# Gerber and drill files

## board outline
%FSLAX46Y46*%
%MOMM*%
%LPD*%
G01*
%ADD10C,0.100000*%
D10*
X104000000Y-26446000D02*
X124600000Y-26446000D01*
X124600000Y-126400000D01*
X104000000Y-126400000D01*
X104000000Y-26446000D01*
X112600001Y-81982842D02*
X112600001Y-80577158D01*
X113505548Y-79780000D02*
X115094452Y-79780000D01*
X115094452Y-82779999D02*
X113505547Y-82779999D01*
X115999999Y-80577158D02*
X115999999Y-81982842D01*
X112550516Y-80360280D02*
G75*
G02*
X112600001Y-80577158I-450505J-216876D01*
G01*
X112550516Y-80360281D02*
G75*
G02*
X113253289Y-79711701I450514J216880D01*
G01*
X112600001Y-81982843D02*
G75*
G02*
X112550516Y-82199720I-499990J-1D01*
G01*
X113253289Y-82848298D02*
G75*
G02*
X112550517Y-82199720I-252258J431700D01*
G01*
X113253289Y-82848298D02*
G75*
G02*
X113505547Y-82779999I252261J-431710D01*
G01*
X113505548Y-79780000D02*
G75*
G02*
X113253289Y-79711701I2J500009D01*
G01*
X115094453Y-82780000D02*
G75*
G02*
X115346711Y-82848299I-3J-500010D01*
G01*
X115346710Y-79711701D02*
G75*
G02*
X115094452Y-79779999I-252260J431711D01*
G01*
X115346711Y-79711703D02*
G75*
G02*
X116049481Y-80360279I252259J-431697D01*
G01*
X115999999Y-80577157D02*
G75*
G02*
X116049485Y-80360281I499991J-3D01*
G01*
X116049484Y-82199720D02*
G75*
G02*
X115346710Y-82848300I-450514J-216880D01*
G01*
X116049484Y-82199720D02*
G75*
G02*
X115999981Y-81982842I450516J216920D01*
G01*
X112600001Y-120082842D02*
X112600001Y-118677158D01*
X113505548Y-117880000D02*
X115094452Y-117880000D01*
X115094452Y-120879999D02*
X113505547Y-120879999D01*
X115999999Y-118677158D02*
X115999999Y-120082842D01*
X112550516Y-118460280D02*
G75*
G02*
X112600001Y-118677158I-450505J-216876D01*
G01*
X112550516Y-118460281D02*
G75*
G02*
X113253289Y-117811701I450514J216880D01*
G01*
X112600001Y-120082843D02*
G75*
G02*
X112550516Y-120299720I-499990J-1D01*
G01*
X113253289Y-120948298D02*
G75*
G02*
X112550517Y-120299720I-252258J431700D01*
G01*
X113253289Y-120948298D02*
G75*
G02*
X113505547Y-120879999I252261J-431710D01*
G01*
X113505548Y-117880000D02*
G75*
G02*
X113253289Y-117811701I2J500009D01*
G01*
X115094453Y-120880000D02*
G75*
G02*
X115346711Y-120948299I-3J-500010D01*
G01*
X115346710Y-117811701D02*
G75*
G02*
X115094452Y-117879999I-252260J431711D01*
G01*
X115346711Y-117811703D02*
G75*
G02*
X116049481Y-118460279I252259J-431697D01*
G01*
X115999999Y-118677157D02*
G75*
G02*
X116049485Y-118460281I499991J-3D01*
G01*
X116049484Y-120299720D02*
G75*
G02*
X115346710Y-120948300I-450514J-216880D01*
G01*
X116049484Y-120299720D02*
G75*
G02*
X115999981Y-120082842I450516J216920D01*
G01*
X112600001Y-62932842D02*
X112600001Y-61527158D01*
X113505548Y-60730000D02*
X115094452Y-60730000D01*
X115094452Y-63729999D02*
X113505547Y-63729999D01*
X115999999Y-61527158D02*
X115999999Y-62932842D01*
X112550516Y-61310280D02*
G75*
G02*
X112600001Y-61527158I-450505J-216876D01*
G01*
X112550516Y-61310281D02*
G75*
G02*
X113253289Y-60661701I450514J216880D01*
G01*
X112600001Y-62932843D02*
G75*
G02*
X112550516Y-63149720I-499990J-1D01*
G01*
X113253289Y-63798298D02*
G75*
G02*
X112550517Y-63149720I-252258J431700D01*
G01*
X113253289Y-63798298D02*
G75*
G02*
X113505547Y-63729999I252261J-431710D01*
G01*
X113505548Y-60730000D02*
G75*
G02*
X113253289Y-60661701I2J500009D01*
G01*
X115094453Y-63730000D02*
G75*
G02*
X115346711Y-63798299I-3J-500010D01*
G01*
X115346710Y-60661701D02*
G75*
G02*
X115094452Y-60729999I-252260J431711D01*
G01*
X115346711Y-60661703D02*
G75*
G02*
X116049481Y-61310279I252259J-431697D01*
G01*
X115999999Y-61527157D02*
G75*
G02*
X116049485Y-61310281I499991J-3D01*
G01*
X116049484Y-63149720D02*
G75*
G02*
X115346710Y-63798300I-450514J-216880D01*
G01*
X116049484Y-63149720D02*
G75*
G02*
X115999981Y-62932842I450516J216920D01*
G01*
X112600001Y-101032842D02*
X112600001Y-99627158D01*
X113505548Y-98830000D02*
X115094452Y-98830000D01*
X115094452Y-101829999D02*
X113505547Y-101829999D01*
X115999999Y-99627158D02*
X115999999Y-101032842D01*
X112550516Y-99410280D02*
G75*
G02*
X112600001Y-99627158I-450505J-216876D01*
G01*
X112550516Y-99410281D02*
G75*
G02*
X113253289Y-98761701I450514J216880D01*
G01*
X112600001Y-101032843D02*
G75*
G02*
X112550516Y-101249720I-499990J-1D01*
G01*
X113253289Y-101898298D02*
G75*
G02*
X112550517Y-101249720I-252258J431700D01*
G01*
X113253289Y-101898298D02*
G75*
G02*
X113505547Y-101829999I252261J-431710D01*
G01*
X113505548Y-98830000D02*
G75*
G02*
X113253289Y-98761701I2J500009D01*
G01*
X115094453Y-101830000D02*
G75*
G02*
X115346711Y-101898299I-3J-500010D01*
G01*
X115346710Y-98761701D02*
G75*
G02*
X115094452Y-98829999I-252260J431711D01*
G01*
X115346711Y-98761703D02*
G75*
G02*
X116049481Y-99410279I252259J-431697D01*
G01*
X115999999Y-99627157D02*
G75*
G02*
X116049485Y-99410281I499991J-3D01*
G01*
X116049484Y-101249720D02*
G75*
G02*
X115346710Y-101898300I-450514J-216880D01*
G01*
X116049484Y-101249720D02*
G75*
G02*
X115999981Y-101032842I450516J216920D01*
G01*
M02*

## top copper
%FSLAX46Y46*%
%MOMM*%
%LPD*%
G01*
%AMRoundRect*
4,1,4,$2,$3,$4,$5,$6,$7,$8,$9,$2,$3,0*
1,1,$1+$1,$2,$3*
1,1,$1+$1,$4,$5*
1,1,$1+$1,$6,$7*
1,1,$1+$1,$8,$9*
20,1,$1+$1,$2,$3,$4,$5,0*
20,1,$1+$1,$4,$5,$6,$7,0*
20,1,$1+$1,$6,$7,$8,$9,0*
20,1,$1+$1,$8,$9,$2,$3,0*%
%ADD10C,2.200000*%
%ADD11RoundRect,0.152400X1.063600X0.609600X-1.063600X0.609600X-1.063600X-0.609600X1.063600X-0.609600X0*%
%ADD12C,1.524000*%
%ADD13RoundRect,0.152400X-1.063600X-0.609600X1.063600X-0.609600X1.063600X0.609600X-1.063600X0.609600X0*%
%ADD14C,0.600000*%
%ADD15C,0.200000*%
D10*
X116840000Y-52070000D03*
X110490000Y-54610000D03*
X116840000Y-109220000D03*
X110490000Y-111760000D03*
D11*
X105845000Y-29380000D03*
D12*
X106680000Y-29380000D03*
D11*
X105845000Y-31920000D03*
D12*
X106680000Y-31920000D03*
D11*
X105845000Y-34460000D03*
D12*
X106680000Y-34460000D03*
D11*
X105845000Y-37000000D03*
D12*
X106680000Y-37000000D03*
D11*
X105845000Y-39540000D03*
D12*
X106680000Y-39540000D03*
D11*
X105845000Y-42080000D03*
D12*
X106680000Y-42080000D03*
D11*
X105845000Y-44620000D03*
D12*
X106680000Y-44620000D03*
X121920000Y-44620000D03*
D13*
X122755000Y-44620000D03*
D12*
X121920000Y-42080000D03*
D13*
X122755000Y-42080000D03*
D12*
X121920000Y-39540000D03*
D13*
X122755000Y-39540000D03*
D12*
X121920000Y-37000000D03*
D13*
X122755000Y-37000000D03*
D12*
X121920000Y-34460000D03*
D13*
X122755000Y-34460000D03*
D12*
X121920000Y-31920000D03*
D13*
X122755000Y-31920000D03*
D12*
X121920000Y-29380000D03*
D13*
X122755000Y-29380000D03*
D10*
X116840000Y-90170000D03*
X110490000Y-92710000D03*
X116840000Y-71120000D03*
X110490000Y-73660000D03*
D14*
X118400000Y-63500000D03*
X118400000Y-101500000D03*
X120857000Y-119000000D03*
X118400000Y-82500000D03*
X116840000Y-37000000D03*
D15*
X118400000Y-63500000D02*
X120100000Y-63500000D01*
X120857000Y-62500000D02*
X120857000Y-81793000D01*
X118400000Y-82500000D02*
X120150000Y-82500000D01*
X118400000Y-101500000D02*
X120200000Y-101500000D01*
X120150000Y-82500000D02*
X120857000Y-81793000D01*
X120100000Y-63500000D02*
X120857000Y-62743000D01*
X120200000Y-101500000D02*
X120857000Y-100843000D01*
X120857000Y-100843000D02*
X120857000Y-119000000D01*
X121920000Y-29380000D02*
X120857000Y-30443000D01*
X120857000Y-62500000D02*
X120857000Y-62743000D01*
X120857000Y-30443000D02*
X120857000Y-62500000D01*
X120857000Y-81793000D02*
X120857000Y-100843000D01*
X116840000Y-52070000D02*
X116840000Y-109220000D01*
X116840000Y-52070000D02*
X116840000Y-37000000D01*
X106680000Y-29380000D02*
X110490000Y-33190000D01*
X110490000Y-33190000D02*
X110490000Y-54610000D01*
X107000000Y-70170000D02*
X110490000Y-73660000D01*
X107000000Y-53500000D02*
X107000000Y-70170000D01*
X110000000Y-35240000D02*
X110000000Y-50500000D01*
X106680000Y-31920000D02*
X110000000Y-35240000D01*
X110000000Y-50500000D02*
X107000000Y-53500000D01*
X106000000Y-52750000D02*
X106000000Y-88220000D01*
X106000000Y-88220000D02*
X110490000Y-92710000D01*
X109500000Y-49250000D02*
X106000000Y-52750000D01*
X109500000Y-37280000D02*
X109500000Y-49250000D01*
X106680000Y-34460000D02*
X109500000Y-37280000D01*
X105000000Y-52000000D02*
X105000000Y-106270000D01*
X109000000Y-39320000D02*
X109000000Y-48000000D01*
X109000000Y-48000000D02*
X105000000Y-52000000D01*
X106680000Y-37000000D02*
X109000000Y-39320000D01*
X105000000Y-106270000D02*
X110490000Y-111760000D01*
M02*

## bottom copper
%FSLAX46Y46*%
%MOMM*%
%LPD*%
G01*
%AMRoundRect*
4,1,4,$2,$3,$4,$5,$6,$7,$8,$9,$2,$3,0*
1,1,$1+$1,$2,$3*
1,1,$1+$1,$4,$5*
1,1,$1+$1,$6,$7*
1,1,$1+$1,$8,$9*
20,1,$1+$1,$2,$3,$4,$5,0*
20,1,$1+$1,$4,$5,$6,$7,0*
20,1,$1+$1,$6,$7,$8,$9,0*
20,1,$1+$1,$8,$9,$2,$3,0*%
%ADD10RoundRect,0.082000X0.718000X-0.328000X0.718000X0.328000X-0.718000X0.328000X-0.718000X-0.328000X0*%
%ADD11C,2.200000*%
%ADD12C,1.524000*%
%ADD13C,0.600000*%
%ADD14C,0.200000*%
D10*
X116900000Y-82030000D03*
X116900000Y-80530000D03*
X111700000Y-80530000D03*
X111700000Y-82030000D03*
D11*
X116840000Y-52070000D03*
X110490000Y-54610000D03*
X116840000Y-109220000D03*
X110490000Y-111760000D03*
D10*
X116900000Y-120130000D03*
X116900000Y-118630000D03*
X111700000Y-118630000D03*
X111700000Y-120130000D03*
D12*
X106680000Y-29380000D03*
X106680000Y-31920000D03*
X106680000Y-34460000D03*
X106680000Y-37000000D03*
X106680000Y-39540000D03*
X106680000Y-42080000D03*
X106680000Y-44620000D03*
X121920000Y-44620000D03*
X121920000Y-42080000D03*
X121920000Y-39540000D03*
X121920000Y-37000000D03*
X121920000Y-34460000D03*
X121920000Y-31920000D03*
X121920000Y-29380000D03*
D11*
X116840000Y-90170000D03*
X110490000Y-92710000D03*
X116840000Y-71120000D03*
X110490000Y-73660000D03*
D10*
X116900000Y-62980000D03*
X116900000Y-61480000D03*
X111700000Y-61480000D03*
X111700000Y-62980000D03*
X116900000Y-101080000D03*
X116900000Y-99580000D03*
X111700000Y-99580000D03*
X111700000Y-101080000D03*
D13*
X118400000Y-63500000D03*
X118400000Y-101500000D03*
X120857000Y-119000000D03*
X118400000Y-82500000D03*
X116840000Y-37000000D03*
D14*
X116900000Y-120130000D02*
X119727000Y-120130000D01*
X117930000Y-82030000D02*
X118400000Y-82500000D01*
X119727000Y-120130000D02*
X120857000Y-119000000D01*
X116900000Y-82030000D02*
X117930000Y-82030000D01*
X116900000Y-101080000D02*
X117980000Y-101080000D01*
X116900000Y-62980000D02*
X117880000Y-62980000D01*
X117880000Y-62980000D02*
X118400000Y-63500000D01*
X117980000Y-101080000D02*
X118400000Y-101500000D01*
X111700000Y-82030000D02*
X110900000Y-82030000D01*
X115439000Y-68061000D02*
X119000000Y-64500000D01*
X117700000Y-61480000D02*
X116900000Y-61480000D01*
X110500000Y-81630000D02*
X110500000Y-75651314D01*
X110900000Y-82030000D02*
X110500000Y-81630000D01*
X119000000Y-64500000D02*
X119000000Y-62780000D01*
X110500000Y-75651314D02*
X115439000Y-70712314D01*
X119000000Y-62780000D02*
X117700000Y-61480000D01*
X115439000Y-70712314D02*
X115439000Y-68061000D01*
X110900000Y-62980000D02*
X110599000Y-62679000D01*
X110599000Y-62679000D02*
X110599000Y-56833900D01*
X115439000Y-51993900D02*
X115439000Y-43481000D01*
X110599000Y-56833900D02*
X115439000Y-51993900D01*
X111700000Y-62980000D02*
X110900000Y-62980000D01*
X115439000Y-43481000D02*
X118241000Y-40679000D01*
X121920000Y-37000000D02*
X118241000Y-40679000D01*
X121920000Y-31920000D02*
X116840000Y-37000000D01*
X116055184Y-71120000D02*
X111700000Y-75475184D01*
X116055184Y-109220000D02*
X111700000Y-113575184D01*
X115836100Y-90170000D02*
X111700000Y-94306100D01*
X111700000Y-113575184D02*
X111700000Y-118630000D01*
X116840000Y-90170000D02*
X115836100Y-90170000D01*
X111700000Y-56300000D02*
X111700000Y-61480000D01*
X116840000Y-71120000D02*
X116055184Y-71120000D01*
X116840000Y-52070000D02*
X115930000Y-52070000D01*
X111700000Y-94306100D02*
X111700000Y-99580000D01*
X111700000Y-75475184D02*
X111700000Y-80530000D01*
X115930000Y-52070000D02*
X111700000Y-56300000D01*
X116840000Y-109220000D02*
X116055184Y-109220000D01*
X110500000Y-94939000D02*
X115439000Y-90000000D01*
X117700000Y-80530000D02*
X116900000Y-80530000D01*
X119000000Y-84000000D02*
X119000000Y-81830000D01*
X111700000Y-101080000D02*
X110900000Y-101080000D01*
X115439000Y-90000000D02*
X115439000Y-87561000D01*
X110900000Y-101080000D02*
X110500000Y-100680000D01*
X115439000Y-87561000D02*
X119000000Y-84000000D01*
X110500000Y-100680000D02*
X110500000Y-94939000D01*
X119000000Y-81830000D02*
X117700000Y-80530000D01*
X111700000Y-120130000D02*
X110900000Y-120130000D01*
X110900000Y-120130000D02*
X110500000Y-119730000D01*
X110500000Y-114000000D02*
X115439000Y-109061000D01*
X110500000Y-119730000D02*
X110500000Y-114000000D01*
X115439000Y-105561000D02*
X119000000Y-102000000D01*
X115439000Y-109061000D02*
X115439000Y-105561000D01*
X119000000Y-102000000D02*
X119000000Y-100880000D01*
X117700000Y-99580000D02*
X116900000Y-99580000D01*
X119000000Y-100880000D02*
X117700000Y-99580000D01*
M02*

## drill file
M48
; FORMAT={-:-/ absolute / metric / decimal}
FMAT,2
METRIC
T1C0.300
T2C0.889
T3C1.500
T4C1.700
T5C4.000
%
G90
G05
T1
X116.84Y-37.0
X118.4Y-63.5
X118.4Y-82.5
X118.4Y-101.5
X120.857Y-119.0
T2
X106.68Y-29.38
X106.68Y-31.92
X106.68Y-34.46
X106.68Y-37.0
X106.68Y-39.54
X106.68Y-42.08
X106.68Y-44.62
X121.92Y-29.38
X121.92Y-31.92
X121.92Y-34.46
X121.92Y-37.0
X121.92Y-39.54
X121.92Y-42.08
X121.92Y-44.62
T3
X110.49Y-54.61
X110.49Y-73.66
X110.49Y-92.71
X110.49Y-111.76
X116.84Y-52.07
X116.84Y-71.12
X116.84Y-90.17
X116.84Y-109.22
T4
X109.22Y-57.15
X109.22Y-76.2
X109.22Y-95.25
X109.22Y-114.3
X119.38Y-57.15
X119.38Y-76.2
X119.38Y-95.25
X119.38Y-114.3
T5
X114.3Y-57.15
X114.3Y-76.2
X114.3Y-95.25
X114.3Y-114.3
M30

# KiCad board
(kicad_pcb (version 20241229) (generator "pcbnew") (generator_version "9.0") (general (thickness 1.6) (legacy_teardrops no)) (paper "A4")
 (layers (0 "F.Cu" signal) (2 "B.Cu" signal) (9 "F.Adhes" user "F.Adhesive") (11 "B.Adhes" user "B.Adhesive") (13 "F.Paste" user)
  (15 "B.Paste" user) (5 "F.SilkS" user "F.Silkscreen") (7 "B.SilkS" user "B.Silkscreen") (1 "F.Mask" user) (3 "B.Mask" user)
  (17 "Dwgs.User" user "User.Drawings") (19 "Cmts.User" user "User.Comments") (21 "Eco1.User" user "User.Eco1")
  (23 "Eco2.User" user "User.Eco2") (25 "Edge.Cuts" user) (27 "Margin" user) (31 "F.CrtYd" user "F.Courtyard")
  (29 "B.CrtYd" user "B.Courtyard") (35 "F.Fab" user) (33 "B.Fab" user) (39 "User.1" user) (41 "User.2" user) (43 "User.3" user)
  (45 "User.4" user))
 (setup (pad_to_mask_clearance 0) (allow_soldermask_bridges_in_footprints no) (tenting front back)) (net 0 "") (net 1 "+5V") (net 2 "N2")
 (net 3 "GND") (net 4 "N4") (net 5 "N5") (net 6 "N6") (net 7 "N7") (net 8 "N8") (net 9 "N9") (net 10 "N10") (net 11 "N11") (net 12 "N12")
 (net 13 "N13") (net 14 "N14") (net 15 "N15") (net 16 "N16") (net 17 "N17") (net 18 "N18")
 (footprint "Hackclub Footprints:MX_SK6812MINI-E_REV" (layer "F.Cu") (at 114.3 76.2)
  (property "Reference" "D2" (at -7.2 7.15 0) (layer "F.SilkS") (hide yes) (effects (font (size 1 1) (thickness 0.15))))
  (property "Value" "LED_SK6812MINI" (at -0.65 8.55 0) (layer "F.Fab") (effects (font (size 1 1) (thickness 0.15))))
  (fp_line (start -1.699999 5.782842) (end -1.699999 4.377158) (stroke (width 0.1) (type solid)) (layer "Edge.Cuts"))
  (fp_line (start -0.794452 3.58) (end 0.794452 3.58) (stroke (width 0.1) (type solid)) (layer "Edge.Cuts"))
  (fp_line (start 0.794452 6.579999) (end -0.794453 6.579999) (stroke (width 0.1) (type solid)) (layer "Edge.Cuts"))
  (fp_line (start 1.699999 4.377158) (end 1.699999 5.782842) (stroke (width 0.1) (type solid)) (layer "Edge.Cuts"))
  (fp_arc (start -1.749484 4.16028) (mid -1.712527 4.265932) (end -1.699999 4.377158) (stroke (width 0.1) (type solid)) (layer "Edge.Cuts"))
  (fp_arc (start -1.749484 4.160281) (mid -1.638072 3.575965) (end -1.046711 3.511701) (stroke (width 0.1) (type solid)) (layer "Edge.Cuts"))
  (fp_arc (start -1.699999 5.782843) (mid -1.712527 5.894068) (end -1.749484 5.99972) (stroke (width 0.1) (type solid)) (layer "Edge.Cuts"))
  (fp_arc (start -1.046711 6.648298) (mid -1.638071 6.584034) (end -1.749484 5.99972) (stroke (width 0.1) (type solid)) (layer "Edge.Cuts"))
  (fp_arc (start -1.046711 6.648298) (mid -0.925123 6.597376) (end -0.794453 6.579999) (stroke (width 0.1) (type solid)) (layer "Edge.Cuts"))
  (fp_arc (start -0.794452 3.58) (mid -0.925123 3.562623) (end -1.046711 3.511701) (stroke (width 0.1) (type solid)) (layer "Edge.Cuts"))
  (fp_arc (start 0.794453 6.58) (mid 0.925123 6.597377) (end 1.046711 6.648299) (stroke (width 0.1) (type solid)) (layer "Edge.Cuts"))
  (fp_arc (start 1.04671 3.511701) (mid 0.925122 3.562623) (end 0.794452 3.58) (stroke (width 0.1) (type solid)) (layer "Edge.Cuts"))
  (fp_arc (start 1.046711 3.511703) (mid 1.63807 3.575966) (end 1.749484 4.16028) (stroke (width 0.1) (type solid)) (layer "Edge.Cuts"))
  (fp_arc (start 1.699999 4.377157) (mid 1.712527 4.265932) (end 1.749484 4.16028) (stroke (width 0.1) (type solid)) (layer "Edge.Cuts"))
  (fp_arc (start 1.749484 5.99972) (mid 1.638071 6.584035) (end 1.046711 6.648299) (stroke (width 0.1) (type solid)) (layer "Edge.Cuts"))
  (fp_arc (start 1.749484 5.99972) (mid 1.712527 5.894068) (end 1.699999 5.782842) (stroke (width 0.1) (type solid)) (layer "Edge.Cuts"))
  (pad "1" smd roundrect (at 2.6 5.83 90) (size 0.82 1.6) (layers "B.Cu" "B.Mask" "B.Paste") (roundrect_rratio 0.1) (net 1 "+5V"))
  (pad "2" smd roundrect (at 2.6 4.33 90) (size 0.82 1.6) (layers "B.Cu" "B.Mask" "B.Paste") (roundrect_rratio 0.1) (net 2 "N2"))
  (pad "3" smd roundrect (at -2.6 4.33 90) (size 0.82 1.6) (layers "B.Cu" "B.Mask" "B.Paste") (roundrect_rratio 0.1) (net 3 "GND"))
  (pad "4" smd roundrect (at -2.6 5.83 90) (size 0.82 1.6) (layers "B.Cu" "B.Mask" "B.Paste") (roundrect_rratio 0.1) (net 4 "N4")))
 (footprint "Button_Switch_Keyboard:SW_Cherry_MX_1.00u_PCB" (layer "F.Cu") (at 116.84 52.07)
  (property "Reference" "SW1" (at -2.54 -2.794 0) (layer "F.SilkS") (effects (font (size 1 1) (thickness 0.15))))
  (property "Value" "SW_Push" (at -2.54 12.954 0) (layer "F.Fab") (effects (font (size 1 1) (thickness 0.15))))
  (pad "" np_thru_hole circle (at -7.62 5.08) (size 1.7 1.7) (drill 1.7) (layers "*.Cu" "*.Mask"))
  (pad "" np_thru_hole circle (at -2.54 5.08) (size 4 4) (drill 4) (layers "*.Cu" "*.Mask"))
  (pad "" np_thru_hole circle (at 2.54 5.08) (size 1.7 1.7) (drill 1.7) (layers "*.Cu" "*.Mask"))
  (pad "1" thru_hole circle (at 0 0) (size 2.2 2.2) (drill 1.5) (layers "*.Cu" "*.Mask") (remove_unused_layers no) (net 3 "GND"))
  (pad "2" thru_hole circle (at -6.35 2.54) (size 2.2 2.2) (drill 1.5) (layers "*.Cu" "*.Mask") (remove_unused_layers no) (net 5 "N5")))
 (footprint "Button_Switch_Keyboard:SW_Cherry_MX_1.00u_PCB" (layer "F.Cu") (at 116.84 109.22)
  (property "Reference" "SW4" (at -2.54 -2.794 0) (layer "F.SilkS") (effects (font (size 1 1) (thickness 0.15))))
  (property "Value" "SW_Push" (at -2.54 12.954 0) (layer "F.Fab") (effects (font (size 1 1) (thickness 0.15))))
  (pad "" np_thru_hole circle (at -7.62 5.08) (size 1.7 1.7) (drill 1.7) (layers "*.Cu" "*.Mask"))
  (pad "" np_thru_hole circle (at -2.54 5.08) (size 4 4) (drill 4) (layers "*.Cu" "*.Mask"))
  (pad "" np_thru_hole circle (at 2.54 5.08) (size 1.7 1.7) (drill 1.7) (layers "*.Cu" "*.Mask"))
  (pad "1" thru_hole circle (at 0 0) (size 2.2 2.2) (drill 1.5) (layers "*.Cu" "*.Mask") (remove_unused_layers no) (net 3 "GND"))
  (pad "2" thru_hole circle (at -6.35 2.54) (size 2.2 2.2) (drill 1.5) (layers "*.Cu" "*.Mask") (remove_unused_layers no) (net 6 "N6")))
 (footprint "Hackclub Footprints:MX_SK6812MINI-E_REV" (layer "F.Cu") (at 114.3 114.3)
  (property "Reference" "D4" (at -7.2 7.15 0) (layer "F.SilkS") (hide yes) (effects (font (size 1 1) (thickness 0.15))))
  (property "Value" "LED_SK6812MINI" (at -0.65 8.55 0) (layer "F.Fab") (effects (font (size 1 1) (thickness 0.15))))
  (fp_line (start -1.699999 5.782842) (end -1.699999 4.377158) (stroke (width 0.1) (type solid)) (layer "Edge.Cuts"))
  (fp_line (start -0.794452 3.58) (end 0.794452 3.58) (stroke (width 0.1) (type solid)) (layer "Edge.Cuts"))
  (fp_line (start 0.794452 6.579999) (end -0.794453 6.579999) (stroke (width 0.1) (type solid)) (layer "Edge.Cuts"))
  (fp_line (start 1.699999 4.377158) (end 1.699999 5.782842) (stroke (width 0.1) (type solid)) (layer "Edge.Cuts"))
  (fp_arc (start -1.749484 4.16028) (mid -1.712527 4.265932) (end -1.699999 4.377158) (stroke (width 0.1) (type solid)) (layer "Edge.Cuts"))
  (fp_arc (start -1.749484 4.160281) (mid -1.638072 3.575965) (end -1.046711 3.511701) (stroke (width 0.1) (type solid)) (layer "Edge.Cuts"))
  (fp_arc (start -1.699999 5.782843) (mid -1.712527 5.894068) (end -1.749484 5.99972) (stroke (width 0.1) (type solid)) (layer "Edge.Cuts"))
  (fp_arc (start -1.046711 6.648298) (mid -1.638071 6.584034) (end -1.749484 5.99972) (stroke (width 0.1) (type solid)) (layer "Edge.Cuts"))
  (fp_arc (start -1.046711 6.648298) (mid -0.925123 6.597376) (end -0.794453 6.579999) (stroke (width 0.1) (type solid)) (layer "Edge.Cuts"))
  (fp_arc (start -0.794452 3.58) (mid -0.925123 3.562623) (end -1.046711 3.511701) (stroke (width 0.1) (type solid)) (layer "Edge.Cuts"))
  (fp_arc (start 0.794453 6.58) (mid 0.925123 6.597377) (end 1.046711 6.648299) (stroke (width 0.1) (type solid)) (layer "Edge.Cuts"))
  (fp_arc (start 1.04671 3.511701) (mid 0.925122 3.562623) (end 0.794452 3.58) (stroke (width 0.1) (type solid)) (layer "Edge.Cuts"))
  (fp_arc (start 1.046711 3.511703) (mid 1.63807 3.575966) (end 1.749484 4.16028) (stroke (width 0.1) (type solid)) (layer "Edge.Cuts"))
  (fp_arc (start 1.699999 4.377157) (mid 1.712527 4.265932) (end 1.749484 4.16028) (stroke (width 0.1) (type solid)) (layer "Edge.Cuts"))
  (fp_arc (start 1.749484 5.99972) (mid 1.638071 6.584035) (end 1.046711 6.648299) (stroke (width 0.1) (type solid)) (layer "Edge.Cuts"))
  (fp_arc (start 1.749484 5.99972) (mid 1.712527 5.894068) (end 1.699999 5.782842) (stroke (width 0.1) (type solid)) (layer "Edge.Cuts"))
  (pad "1" smd roundrect (at 2.6 5.83 90) (size 0.82 1.6) (layers "B.Cu" "B.Mask" "B.Paste") (roundrect_rratio 0.1) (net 1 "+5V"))
  (pad "2" smd roundrect (at 2.6 4.33 90) (size 0.82 1.6) (layers "B.Cu" "B.Mask" "B.Paste") (roundrect_rratio 0.1) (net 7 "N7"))
  (pad "3" smd roundrect (at -2.6 4.33 90) (size 0.82 1.6) (layers "B.Cu" "B.Mask" "B.Paste") (roundrect_rratio 0.1) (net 3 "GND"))
  (pad "4" smd roundrect (at -2.6 5.83 90) (size 0.82 1.6) (layers "B.Cu" "B.Mask" "B.Paste") (roundrect_rratio 0.1) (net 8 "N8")))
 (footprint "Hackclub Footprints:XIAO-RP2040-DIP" (layer "F.Cu") (at 114.3 37)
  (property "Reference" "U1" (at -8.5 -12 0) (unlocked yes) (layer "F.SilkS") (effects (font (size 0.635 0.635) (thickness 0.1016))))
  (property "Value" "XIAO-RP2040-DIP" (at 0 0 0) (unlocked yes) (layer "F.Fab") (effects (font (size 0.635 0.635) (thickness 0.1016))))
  (pad "1" smd roundrect (at -8.455 -7.62 180) (size 2.432 1.524) (layers "F.Cu" "F.Mask") (roundrect_rratio 0.1) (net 5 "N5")
   (thermal_bridge_angle 45))
  (pad "1" thru_hole circle (at -7.62 -7.62 180) (size 1.524 1.524) (drill 0.889) (layers "*.Cu" "*.Mask") (remove_unused_layers no)
   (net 5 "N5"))
  (pad "2" smd roundrect (at -8.455 -5.08 180) (size 2.432 1.524) (layers "F.Cu" "F.Mask") (roundrect_rratio 0.1) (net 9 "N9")
   (thermal_bridge_angle 45))
  (pad "2" thru_hole circle (at -7.62 -5.08 180) (size 1.524 1.524) (drill 0.889) (layers "*.Cu" "*.Mask") (remove_unused_layers no)
   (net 9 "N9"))
  (pad "3" smd roundrect (at -8.455 -2.54 180) (size 2.432 1.524) (layers "F.Cu" "F.Mask") (roundrect_rratio 0.1) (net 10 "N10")
   (thermal_bridge_angle 45))
  (pad "3" thru_hole circle (at -7.62 -2.54 180) (size 1.524 1.524) (drill 0.889) (layers "*.Cu" "*.Mask") (remove_unused_layers no)
   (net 10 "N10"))
  (pad "4" smd roundrect (at -8.455 0 180) (size 2.432 1.524) (layers "F.Cu" "F.Mask") (roundrect_rratio 0.1) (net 6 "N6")
   (thermal_bridge_angle 45))
  (pad "4" thru_hole circle (at -7.62 0 180) (size 1.524 1.524) (drill 0.889) (layers "*.Cu" "*.Mask") (remove_unused_layers no)
   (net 6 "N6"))
  (pad "5" smd roundrect (at -8.455 2.54 180) (size 2.432 1.524) (layers "F.Cu" "F.Mask") (roundrect_rratio 0.1) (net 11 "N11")
   (thermal_bridge_angle 45))
  (pad "5" thru_hole circle (at -7.62 2.54 180) (size 1.524 1.524) (drill 0.889) (layers "*.Cu" "*.Mask") (remove_unused_layers no)
   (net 11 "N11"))
  (pad "6" smd roundrect (at -8.455 5.08 180) (size 2.432 1.524) (layers "F.Cu" "F.Mask") (roundrect_rratio 0.1) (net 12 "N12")
   (thermal_bridge_angle 45))
  (pad "6" thru_hole circle (at -7.62 5.08 180) (size 1.524 1.524) (drill 0.889) (layers "*.Cu" "*.Mask") (remove_unused_layers no)
   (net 12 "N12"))
  (pad "7" smd roundrect (at -8.455 7.62 180) (size 2.432 1.524) (layers "F.Cu" "F.Mask") (roundrect_rratio 0.1) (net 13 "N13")
   (thermal_bridge_angle 45))
  (pad "7" thru_hole circle (at -7.62 7.62 180) (size 1.524 1.524) (drill 0.889) (layers "*.Cu" "*.Mask") (remove_unused_layers no)
   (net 13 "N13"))
  (pad "8" thru_hole circle (at 7.62 7.62) (size 1.524 1.524) (drill 0.889) (layers "*.Cu" "*.Mask") (remove_unused_layers no)
   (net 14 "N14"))
  (pad "8" smd roundrect (at 8.455 7.62) (size 2.432 1.524) (layers "F.Cu" "F.Mask") (roundrect_rratio 0.1) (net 14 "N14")
   (thermal_bridge_angle 45))
  (pad "9" thru_hole circle (at 7.62 5.08) (size 1.524 1.524) (drill 0.889) (layers "*.Cu" "*.Mask") (remove_unused_layers no)
   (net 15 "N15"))
  (pad "9" smd roundrect (at 8.455 5.08) (size 2.432 1.524) (layers "F.Cu" "F.Mask") (roundrect_rratio 0.1) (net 15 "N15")
   (thermal_bridge_angle 45))
  (pad "10" thru_hole circle (at 7.62 2.54) (size 1.524 1.524) (drill 0.889) (layers "*.Cu" "*.Mask") (remove_unused_layers no)
   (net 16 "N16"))
  (pad "10" smd roundrect (at 8.455 2.54) (size 2.432 1.524) (layers "F.Cu" "F.Mask") (roundrect_rratio 0.1) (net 16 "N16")
   (thermal_bridge_angle 45))
  (pad "11" thru_hole circle (at 7.62 0) (size 1.524 1.524) (drill 0.889) (layers "*.Cu" "*.Mask") (remove_unused_layers no) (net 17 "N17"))
  (pad "11" smd roundrect (at 8.455 0) (size 2.432 1.524) (layers "F.Cu" "F.Mask") (roundrect_rratio 0.1) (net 17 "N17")
   (thermal_bridge_angle 45))
  (pad "12" thru_hole circle (at 7.62 -2.54) (size 1.524 1.524) (drill 0.889) (layers "*.Cu" "*.Mask") (remove_unused_layers no)
   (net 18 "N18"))
  (pad "12" smd roundrect (at 8.455 -2.54) (size 2.432 1.524) (layers "F.Cu" "F.Mask") (roundrect_rratio 0.1) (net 18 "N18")
   (thermal_bridge_angle 45))
  (pad "13" thru_hole circle (at 7.62 -5.08) (size 1.524 1.524) (drill 0.889) (layers "*.Cu" "*.Mask") (remove_unused_layers no)
   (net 3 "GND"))
  (pad "13" smd roundrect (at 8.455 -5.08) (size 2.432 1.524) (layers "F.Cu" "F.Mask") (roundrect_rratio 0.1) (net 3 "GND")
   (thermal_bridge_angle 45))
  (pad "14" thru_hole circle (at 7.62 -7.62) (size 1.524 1.524) (drill 0.889) (layers "*.Cu" "*.Mask") (remove_unused_layers no)
   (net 1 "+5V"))
  (pad "14" smd roundrect (at 8.455 -7.62) (size 2.432 1.524) (layers "F.Cu" "F.Mask") (roundrect_rratio 0.1) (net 1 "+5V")
   (thermal_bridge_angle 45)))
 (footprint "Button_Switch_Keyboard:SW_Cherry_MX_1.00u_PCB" (layer "F.Cu") (at 116.84 90.17)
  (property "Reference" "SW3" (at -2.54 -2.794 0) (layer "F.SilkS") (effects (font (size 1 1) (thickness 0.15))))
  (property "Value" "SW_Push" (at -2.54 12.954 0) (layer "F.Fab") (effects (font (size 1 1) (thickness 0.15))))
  (pad "" np_thru_hole circle (at -7.62 5.08) (size 1.7 1.7) (drill 1.7) (layers "*.Cu" "*.Mask"))
  (pad "" np_thru_hole circle (at -2.54 5.08) (size 4 4) (drill 4) (layers "*.Cu" "*.Mask"))
  (pad "" np_thru_hole circle (at 2.54 5.08) (size 1.7 1.7) (drill 1.7) (layers "*.Cu" "*.Mask"))
  (pad "1" thru_hole circle (at 0 0) (size 2.2 2.2) (drill 1.5) (layers "*.Cu" "*.Mask") (remove_unused_layers no) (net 3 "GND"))
  (pad "2" thru_hole circle (at -6.35 2.54) (size 2.2 2.2) (drill 1.5) (layers "*.Cu" "*.Mask") (remove_unused_layers no) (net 10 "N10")))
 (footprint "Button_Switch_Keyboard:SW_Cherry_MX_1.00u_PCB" (layer "F.Cu") (at 116.84 71.12)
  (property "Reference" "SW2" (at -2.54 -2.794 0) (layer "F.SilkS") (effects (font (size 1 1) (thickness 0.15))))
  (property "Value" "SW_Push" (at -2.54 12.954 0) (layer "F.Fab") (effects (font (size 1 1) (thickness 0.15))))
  (pad "" np_thru_hole circle (at -7.62 5.08) (size 1.7 1.7) (drill 1.7) (layers "*.Cu" "*.Mask"))
  (pad "" np_thru_hole circle (at -2.54 5.08) (size 4 4) (drill 4) (layers "*.Cu" "*.Mask"))
  (pad "" np_thru_hole circle (at 2.54 5.08) (size 1.7 1.7) (drill 1.7) (layers "*.Cu" "*.Mask"))
  (pad "1" thru_hole circle (at 0 0) (size 2.2 2.2) (drill 1.5) (layers "*.Cu" "*.Mask") (remove_unused_layers no) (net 3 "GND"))
  (pad "2" thru_hole circle (at -6.35 2.54) (size 2.2 2.2) (drill 1.5) (layers "*.Cu" "*.Mask") (remove_unused_layers no) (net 9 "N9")))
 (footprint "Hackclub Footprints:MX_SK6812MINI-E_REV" (layer "F.Cu") (at 114.3 57.15)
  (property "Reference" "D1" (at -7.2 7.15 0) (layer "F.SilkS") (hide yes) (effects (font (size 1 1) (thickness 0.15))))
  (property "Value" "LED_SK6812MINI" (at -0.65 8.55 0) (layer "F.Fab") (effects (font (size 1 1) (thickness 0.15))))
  (fp_line (start -1.699999 5.782842) (end -1.699999 4.377158) (stroke (width 0.1) (type solid)) (layer "Edge.Cuts"))
  (fp_line (start -0.794452 3.58) (end 0.794452 3.58) (stroke (width 0.1) (type solid)) (layer "Edge.Cuts"))
  (fp_line (start 0.794452 6.579999) (end -0.794453 6.579999) (stroke (width 0.1) (type solid)) (layer "Edge.Cuts"))
  (fp_line (start 1.699999 4.377158) (end 1.699999 5.782842) (stroke (width 0.1) (type solid)) (layer "Edge.Cuts"))
  (fp_arc (start -1.749484 4.16028) (mid -1.712527 4.265932) (end -1.699999 4.377158) (stroke (width 0.1) (type solid)) (layer "Edge.Cuts"))
  (fp_arc (start -1.749484 4.160281) (mid -1.638072 3.575965) (end -1.046711 3.511701) (stroke (width 0.1) (type solid)) (layer "Edge.Cuts"))
  (fp_arc (start -1.699999 5.782843) (mid -1.712527 5.894068) (end -1.749484 5.99972) (stroke (width 0.1) (type solid)) (layer "Edge.Cuts"))
  (fp_arc (start -1.046711 6.648298) (mid -1.638071 6.584034) (end -1.749484 5.99972) (stroke (width 0.1) (type solid)) (layer "Edge.Cuts"))
  (fp_arc (start -1.046711 6.648298) (mid -0.925123 6.597376) (end -0.794453 6.579999) (stroke (width 0.1) (type solid)) (layer "Edge.Cuts"))
  (fp_arc (start -0.794452 3.58) (mid -0.925123 3.562623) (end -1.046711 3.511701) (stroke (width 0.1) (type solid)) (layer "Edge.Cuts"))
  (fp_arc (start 0.794453 6.58) (mid 0.925123 6.597377) (end 1.046711 6.648299) (stroke (width 0.1) (type solid)) (layer "Edge.Cuts"))
  (fp_arc (start 1.04671 3.511701) (mid 0.925122 3.562623) (end 0.794452 3.58) (stroke (width 0.1) (type solid)) (layer "Edge.Cuts"))
  (fp_arc (start 1.046711 3.511703) (mid 1.63807 3.575966) (end 1.749484 4.16028) (stroke (width 0.1) (type solid)) (layer "Edge.Cuts"))
  (fp_arc (start 1.699999 4.377157) (mid 1.712527 4.265932) (end 1.749484 4.16028) (stroke (width 0.1) (type solid)) (layer "Edge.Cuts"))
  (fp_arc (start 1.749484 5.99972) (mid 1.638071 6.584035) (end 1.046711 6.648299) (stroke (width 0.1) (type solid)) (layer "Edge.Cuts"))
  (fp_arc (start 1.749484 5.99972) (mid 1.712527 5.894068) (end 1.699999 5.782842) (stroke (width 0.1) (type solid)) (layer "Edge.Cuts"))
  (pad "1" smd roundrect (at 2.6 5.83 90) (size 0.82 1.6) (layers "B.Cu" "B.Mask" "B.Paste") (roundrect_rratio 0.1) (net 1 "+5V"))
  (pad "2" smd roundrect (at 2.6 4.33 90) (size 0.82 1.6) (layers "B.Cu" "B.Mask" "B.Paste") (roundrect_rratio 0.1) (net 4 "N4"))
  (pad "3" smd roundrect (at -2.6 4.33 90) (size 0.82 1.6) (layers "B.Cu" "B.Mask" "B.Paste") (roundrect_rratio 0.1) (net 3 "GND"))
  (pad "4" smd roundrect (at -2.6 5.83 90) (size 0.82 1.6) (layers "B.Cu" "B.Mask" "B.Paste") (roundrect_rratio 0.1) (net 17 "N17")))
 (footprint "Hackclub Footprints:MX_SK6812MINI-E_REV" (layer "F.Cu") (at 114.3 95.25)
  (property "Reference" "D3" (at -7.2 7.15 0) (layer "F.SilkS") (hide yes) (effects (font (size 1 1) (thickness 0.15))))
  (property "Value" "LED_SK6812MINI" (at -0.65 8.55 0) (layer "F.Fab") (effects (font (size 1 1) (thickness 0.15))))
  (fp_line (start -1.699999 5.782842) (end -1.699999 4.377158) (stroke (width 0.1) (type solid)) (layer "Edge.Cuts"))
  (fp_line (start -0.794452 3.58) (end 0.794452 3.58) (stroke (width 0.1) (type solid)) (layer "Edge.Cuts"))
  (fp_line (start 0.794452 6.579999) (end -0.794453 6.579999) (stroke (width 0.1) (type solid)) (layer "Edge.Cuts"))
  (fp_line (start 1.699999 4.377158) (end 1.699999 5.782842) (stroke (width 0.1) (type solid)) (layer "Edge.Cuts"))
  (fp_arc (start -1.749484 4.16028) (mid -1.712527 4.265932) (end -1.699999 4.377158) (stroke (width 0.1) (type solid)) (layer "Edge.Cuts"))
  (fp_arc (start -1.749484 4.160281) (mid -1.638072 3.575965) (end -1.046711 3.511701) (stroke (width 0.1) (type solid)) (layer "Edge.Cuts"))
  (fp_arc (start -1.699999 5.782843) (mid -1.712527 5.894068) (end -1.749484 5.99972) (stroke (width 0.1) (type solid)) (layer "Edge.Cuts"))
  (fp_arc (start -1.046711 6.648298) (mid -1.638071 6.584034) (end -1.749484 5.99972) (stroke (width 0.1) (type solid)) (layer "Edge.Cuts"))
  (fp_arc (start -1.046711 6.648298) (mid -0.925123 6.597376) (end -0.794453 6.579999) (stroke (width 0.1) (type solid)) (layer "Edge.Cuts"))
  (fp_arc (start -0.794452 3.58) (mid -0.925123 3.562623) (end -1.046711 3.511701) (stroke (width 0.1) (type solid)) (layer "Edge.Cuts"))
  (fp_arc (start 0.794453 6.58) (mid 0.925123 6.597377) (end 1.046711 6.648299) (stroke (width 0.1) (type solid)) (layer "Edge.Cuts"))
  (fp_arc (start 1.04671 3.511701) (mid 0.925122 3.562623) (end 0.794452 3.58) (stroke (width 0.1) (type solid)) (layer "Edge.Cuts"))
  (fp_arc (start 1.046711 3.511703) (mid 1.63807 3.575966) (end 1.749484 4.16028) (stroke (width 0.1) (type solid)) (layer "Edge.Cuts"))
  (fp_arc (start 1.699999 4.377157) (mid 1.712527 4.265932) (end 1.749484 4.16028) (stroke (width 0.1) (type solid)) (layer "Edge.Cuts"))
  (fp_arc (start 1.749484 5.99972) (mid 1.638071 6.584035) (end 1.046711 6.648299) (stroke (width 0.1) (type solid)) (layer "Edge.Cuts"))
  (fp_arc (start 1.749484 5.99972) (mid 1.712527 5.894068) (end 1.699999 5.782842) (stroke (width 0.1) (type solid)) (layer "Edge.Cuts"))
  (pad "1" smd roundrect (at 2.6 5.83 90) (size 0.82 1.6) (layers "B.Cu" "B.Mask" "B.Paste") (roundrect_rratio 0.1) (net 1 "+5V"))
  (pad "2" smd roundrect (at 2.6 4.33 90) (size 0.82 1.6) (layers "B.Cu" "B.Mask" "B.Paste") (roundrect_rratio 0.1) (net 8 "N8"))
  (pad "3" smd roundrect (at -2.6 4.33 90) (size 0.82 1.6) (layers "B.Cu" "B.Mask" "B.Paste") (roundrect_rratio 0.1) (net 3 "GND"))
  (pad "4" smd roundrect (at -2.6 5.83 90) (size 0.82 1.6) (layers "B.Cu" "B.Mask" "B.Paste") (roundrect_rratio 0.1) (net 2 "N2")))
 (gr_rect (start 104 26.446) (end 124.6 126.4) (stroke (width 0.1) (type solid)) (fill no) (layer "Edge.Cuts"))
 (segment (start 118.4 63.5) (end 120.1 63.5) (width 0.2) (layer "F.Cu") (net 1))
 (segment (start 120.857 62.5) (end 120.857 81.793) (width 0.2) (layer "F.Cu") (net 1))
 (segment (start 118.4 82.5) (end 120.15 82.5) (width 0.2) (layer "F.Cu") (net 1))
 (segment (start 118.4 101.5) (end 120.2 101.5) (width 0.2) (layer "F.Cu") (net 1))
 (segment (start 120.15 82.5) (end 120.857 81.793) (width 0.2) (layer "F.Cu") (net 1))
 (segment (start 120.1 63.5) (end 120.857 62.743) (width 0.2) (layer "F.Cu") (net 1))
 (segment (start 120.2 101.5) (end 120.857 100.843) (width 0.2) (layer "F.Cu") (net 1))
 (segment (start 120.857 100.843) (end 120.857 119) (width 0.2) (layer "F.Cu") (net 1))
 (segment (start 121.92 29.38) (end 120.857 30.443) (width 0.2) (layer "F.Cu") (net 1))
 (segment (start 120.857 62.5) (end 120.857 62.743) (width 0.2) (layer "F.Cu") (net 1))
 (segment (start 120.857 30.443) (end 120.857 62.5) (width 0.2) (layer "F.Cu") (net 1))
 (segment (start 120.857 81.793) (end 120.857 100.843) (width 0.2) (layer "F.Cu") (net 1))
 (via (at 118.4 63.5) (size 0.6) (drill 0.3) (layers "F.Cu" "B.Cu") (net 1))
 (via (at 118.4 101.5) (size 0.6) (drill 0.3) (layers "F.Cu" "B.Cu") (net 1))
 (via (at 120.857 119) (size 0.6) (drill 0.3) (layers "F.Cu" "B.Cu") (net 1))
 (via (at 118.4 82.5) (size 0.6) (drill 0.3) (layers "F.Cu" "B.Cu") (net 1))
 (segment (start 116.9 120.13) (end 119.727 120.13) (width 0.2) (layer "B.Cu") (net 1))
 (segment (start 117.93 82.03) (end 118.4 82.5) (width 0.2) (layer "B.Cu") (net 1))
 (segment (start 119.727 120.13) (end 120.857 119) (width 0.2) (layer "B.Cu") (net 1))
 (segment (start 116.9 82.03) (end 117.93 82.03) (width 0.2) (layer "B.Cu") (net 1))
 (segment (start 116.9 101.08) (end 117.98 101.08) (width 0.2) (layer "B.Cu") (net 1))
 (segment (start 116.9 62.98) (end 117.88 62.98) (width 0.2) (layer "B.Cu") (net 1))
 (segment (start 117.88 62.98) (end 118.4 63.5) (width 0.2) (layer "B.Cu") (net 1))
 (segment (start 117.98 101.08) (end 118.4 101.5) (width 0.2) (layer "B.Cu") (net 1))
 (segment (start 111.7 82.03) (end 110.9 82.03) (width 0.2) (layer "B.Cu") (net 4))
 (segment (start 115.439 68.061) (end 119 64.5) (width 0.2) (layer "B.Cu") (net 4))
 (segment (start 117.7 61.48) (end 116.9 61.48) (width 0.2) (layer "B.Cu") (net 4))
 (segment (start 110.5 81.63) (end 110.5 75.651314) (width 0.2) (layer "B.Cu") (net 4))
 (segment (start 110.9 82.03) (end 110.5 81.63) (width 0.2) (layer "B.Cu") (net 4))
 (segment (start 119 64.5) (end 119 62.78) (width 0.2) (layer "B.Cu") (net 4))
 (segment (start 110.5 75.651314) (end 115.439 70.712314) (width 0.2) (layer "B.Cu") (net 4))
 (segment (start 119 62.78) (end 117.7 61.48) (width 0.2) (layer "B.Cu") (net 4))
 (segment (start 115.439 70.712314) (end 115.439 68.061) (width 0.2) (layer "B.Cu") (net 4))
 (segment (start 110.9 62.98) (end 110.599 62.679) (width 0.2) (layer "B.Cu") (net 17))
 (segment (start 110.599 62.679) (end 110.599 56.8339) (width 0.2) (layer "B.Cu") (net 17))
 (segment (start 115.439 51.9939) (end 115.439 43.481) (width 0.2) (layer "B.Cu") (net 17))
 (segment (start 110.599 56.8339) (end 115.439 51.9939) (width 0.2) (layer "B.Cu") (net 17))
 (segment (start 111.7 62.98) (end 110.9 62.98) (width 0.2) (layer "B.Cu") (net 17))
 (segment (start 115.439 43.481) (end 118.241 40.679) (width 0.2) (layer "B.Cu") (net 17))
 (segment (start 121.92 37) (end 118.241 40.679) (width 0.2) (layer "B.Cu") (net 17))
 (segment (start 116.84 52.07) (end 116.84 109.22) (width 0.2) (layer "F.Cu") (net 3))
 (segment (start 116.84 52.07) (end 116.84 37) (width 0.2) (layer "F.Cu") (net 3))
 (via (at 116.84 37) (size 0.6) (drill 0.3) (layers "F.Cu" "B.Cu") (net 3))
 (segment (start 121.92 31.92) (end 116.84 37) (width 0.2) (layer "B.Cu") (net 3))
 (segment (start 116.055184 71.12) (end 111.7 75.475184) (width 0.2) (layer "B.Cu") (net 3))
 (segment (start 116.055184 109.22) (end 111.7 113.575184) (width 0.2) (layer "B.Cu") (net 3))
 (segment (start 115.8361 90.17) (end 111.7 94.3061) (width 0.2) (layer "B.Cu") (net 3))
 (segment (start 111.7 113.575184) (end 111.7 118.63) (width 0.2) (layer "B.Cu") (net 3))
 (segment (start 116.84 90.17) (end 115.8361 90.17) (width 0.2) (layer "B.Cu") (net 3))
 (segment (start 111.7 56.3) (end 111.7 61.48) (width 0.2) (layer "B.Cu") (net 3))
 (segment (start 116.84 71.12) (end 116.055184 71.12) (width 0.2) (layer "B.Cu") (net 3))
 (segment (start 116.84 52.07) (end 115.93 52.07) (width 0.2) (layer "B.Cu") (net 3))
 (segment (start 111.7 94.3061) (end 111.7 99.58) (width 0.2) (layer "B.Cu") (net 3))
 (segment (start 111.7 75.475184) (end 111.7 80.53) (width 0.2) (layer "B.Cu") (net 3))
 (segment (start 115.93 52.07) (end 111.7 56.3) (width 0.2) (layer "B.Cu") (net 3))
 (segment (start 116.84 109.22) (end 116.055184 109.22) (width 0.2) (layer "B.Cu") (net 3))
 (segment (start 110.5 94.939) (end 115.439 90) (width 0.2) (layer "B.Cu") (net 2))
 (segment (start 117.7 80.53) (end 116.9 80.53) (width 0.2) (layer "B.Cu") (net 2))
 (segment (start 119 84) (end 119 81.83) (width 0.2) (layer "B.Cu") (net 2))
 (segment (start 111.7 101.08) (end 110.9 101.08) (width 0.2) (layer "B.Cu") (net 2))
 (segment (start 115.439 90) (end 115.439 87.561) (width 0.2) (layer "B.Cu") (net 2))
 (segment (start 110.9 101.08) (end 110.5 100.68) (width 0.2) (layer "B.Cu") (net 2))
 (segment (start 115.439 87.561) (end 119 84) (width 0.2) (layer "B.Cu") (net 2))
 (segment (start 110.5 100.68) (end 110.5 94.939) (width 0.2) (layer "B.Cu") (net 2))
 (segment (start 119 81.83) (end 117.7 80.53) (width 0.2) (layer "B.Cu") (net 2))
 (segment (start 111.7 120.13) (end 110.9 120.13) (width 0.2) (layer "B.Cu") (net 8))
 (segment (start 110.9 120.13) (end 110.5 119.73) (width 0.2) (layer "B.Cu") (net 8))
 (segment (start 110.5 114) (end 115.439 109.061) (width 0.2) (layer "B.Cu") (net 8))
 (segment (start 110.5 119.73) (end 110.5 114) (width 0.2) (layer "B.Cu") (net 8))
 (segment (start 115.439 105.561) (end 119 102) (width 0.2) (layer "B.Cu") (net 8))
 (segment (start 115.439 109.061) (end 115.439 105.561) (width 0.2) (layer "B.Cu") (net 8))
 (segment (start 119 102) (end 119 100.88) (width 0.2) (layer "B.Cu") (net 8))
 (segment (start 117.7 99.58) (end 116.9 99.58) (width 0.2) (layer "B.Cu") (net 8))
 (segment (start 119 100.88) (end 117.7 99.58) (width 0.2) (layer "B.Cu") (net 8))
 (segment (start 106.68 29.38) (end 110.49 33.19) (width 0.2) (layer "F.Cu") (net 5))
 (segment (start 110.49 33.19) (end 110.49 54.61) (width 0.2) (layer "F.Cu") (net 5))
 (segment (start 107 70.17) (end 110.49 73.66) (width 0.2) (layer "F.Cu") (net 9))
 (segment (start 107 53.5) (end 107 70.17) (width 0.2) (layer "F.Cu") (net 9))
 (segment (start 110 35.24) (end 110 50.5) (width 0.2) (layer "F.Cu") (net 9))
 (segment (start 106.68 31.92) (end 110 35.24) (width 0.2) (layer "F.Cu") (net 9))
 (segment (start 110 50.5) (end 107 53.5) (width 0.2) (layer "F.Cu") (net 9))
 (segment (start 106 52.75) (end 106 88.22) (width 0.2) (layer "F.Cu") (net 10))
 (segment (start 106 88.22) (end 110.49 92.71) (width 0.2) (layer "F.Cu") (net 10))
 (segment (start 109.5 49.25) (end 106 52.75) (width 0.2) (layer "F.Cu") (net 10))
 (segment (start 109.5 37.28) (end 109.5 49.25) (width 0.2) (layer "F.Cu") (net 10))
 (segment (start 106.68 34.46) (end 109.5 37.28) (width 0.2) (layer "F.Cu") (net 10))
 (segment (start 105 52) (end 105 106.27) (width 0.2) (layer "F.Cu") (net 6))
 (segment (start 109 39.32) (end 109 48) (width 0.2) (layer "F.Cu") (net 6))
 (segment (start 109 48) (end 105 52) (width 0.2) (layer "F.Cu") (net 6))
 (segment (start 106.68 37) (end 109 39.32) (width 0.2) (layer "F.Cu") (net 6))
 (segment (start 105 106.27) (end 110.49 111.76) (width 0.2) (layer "F.Cu") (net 6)))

